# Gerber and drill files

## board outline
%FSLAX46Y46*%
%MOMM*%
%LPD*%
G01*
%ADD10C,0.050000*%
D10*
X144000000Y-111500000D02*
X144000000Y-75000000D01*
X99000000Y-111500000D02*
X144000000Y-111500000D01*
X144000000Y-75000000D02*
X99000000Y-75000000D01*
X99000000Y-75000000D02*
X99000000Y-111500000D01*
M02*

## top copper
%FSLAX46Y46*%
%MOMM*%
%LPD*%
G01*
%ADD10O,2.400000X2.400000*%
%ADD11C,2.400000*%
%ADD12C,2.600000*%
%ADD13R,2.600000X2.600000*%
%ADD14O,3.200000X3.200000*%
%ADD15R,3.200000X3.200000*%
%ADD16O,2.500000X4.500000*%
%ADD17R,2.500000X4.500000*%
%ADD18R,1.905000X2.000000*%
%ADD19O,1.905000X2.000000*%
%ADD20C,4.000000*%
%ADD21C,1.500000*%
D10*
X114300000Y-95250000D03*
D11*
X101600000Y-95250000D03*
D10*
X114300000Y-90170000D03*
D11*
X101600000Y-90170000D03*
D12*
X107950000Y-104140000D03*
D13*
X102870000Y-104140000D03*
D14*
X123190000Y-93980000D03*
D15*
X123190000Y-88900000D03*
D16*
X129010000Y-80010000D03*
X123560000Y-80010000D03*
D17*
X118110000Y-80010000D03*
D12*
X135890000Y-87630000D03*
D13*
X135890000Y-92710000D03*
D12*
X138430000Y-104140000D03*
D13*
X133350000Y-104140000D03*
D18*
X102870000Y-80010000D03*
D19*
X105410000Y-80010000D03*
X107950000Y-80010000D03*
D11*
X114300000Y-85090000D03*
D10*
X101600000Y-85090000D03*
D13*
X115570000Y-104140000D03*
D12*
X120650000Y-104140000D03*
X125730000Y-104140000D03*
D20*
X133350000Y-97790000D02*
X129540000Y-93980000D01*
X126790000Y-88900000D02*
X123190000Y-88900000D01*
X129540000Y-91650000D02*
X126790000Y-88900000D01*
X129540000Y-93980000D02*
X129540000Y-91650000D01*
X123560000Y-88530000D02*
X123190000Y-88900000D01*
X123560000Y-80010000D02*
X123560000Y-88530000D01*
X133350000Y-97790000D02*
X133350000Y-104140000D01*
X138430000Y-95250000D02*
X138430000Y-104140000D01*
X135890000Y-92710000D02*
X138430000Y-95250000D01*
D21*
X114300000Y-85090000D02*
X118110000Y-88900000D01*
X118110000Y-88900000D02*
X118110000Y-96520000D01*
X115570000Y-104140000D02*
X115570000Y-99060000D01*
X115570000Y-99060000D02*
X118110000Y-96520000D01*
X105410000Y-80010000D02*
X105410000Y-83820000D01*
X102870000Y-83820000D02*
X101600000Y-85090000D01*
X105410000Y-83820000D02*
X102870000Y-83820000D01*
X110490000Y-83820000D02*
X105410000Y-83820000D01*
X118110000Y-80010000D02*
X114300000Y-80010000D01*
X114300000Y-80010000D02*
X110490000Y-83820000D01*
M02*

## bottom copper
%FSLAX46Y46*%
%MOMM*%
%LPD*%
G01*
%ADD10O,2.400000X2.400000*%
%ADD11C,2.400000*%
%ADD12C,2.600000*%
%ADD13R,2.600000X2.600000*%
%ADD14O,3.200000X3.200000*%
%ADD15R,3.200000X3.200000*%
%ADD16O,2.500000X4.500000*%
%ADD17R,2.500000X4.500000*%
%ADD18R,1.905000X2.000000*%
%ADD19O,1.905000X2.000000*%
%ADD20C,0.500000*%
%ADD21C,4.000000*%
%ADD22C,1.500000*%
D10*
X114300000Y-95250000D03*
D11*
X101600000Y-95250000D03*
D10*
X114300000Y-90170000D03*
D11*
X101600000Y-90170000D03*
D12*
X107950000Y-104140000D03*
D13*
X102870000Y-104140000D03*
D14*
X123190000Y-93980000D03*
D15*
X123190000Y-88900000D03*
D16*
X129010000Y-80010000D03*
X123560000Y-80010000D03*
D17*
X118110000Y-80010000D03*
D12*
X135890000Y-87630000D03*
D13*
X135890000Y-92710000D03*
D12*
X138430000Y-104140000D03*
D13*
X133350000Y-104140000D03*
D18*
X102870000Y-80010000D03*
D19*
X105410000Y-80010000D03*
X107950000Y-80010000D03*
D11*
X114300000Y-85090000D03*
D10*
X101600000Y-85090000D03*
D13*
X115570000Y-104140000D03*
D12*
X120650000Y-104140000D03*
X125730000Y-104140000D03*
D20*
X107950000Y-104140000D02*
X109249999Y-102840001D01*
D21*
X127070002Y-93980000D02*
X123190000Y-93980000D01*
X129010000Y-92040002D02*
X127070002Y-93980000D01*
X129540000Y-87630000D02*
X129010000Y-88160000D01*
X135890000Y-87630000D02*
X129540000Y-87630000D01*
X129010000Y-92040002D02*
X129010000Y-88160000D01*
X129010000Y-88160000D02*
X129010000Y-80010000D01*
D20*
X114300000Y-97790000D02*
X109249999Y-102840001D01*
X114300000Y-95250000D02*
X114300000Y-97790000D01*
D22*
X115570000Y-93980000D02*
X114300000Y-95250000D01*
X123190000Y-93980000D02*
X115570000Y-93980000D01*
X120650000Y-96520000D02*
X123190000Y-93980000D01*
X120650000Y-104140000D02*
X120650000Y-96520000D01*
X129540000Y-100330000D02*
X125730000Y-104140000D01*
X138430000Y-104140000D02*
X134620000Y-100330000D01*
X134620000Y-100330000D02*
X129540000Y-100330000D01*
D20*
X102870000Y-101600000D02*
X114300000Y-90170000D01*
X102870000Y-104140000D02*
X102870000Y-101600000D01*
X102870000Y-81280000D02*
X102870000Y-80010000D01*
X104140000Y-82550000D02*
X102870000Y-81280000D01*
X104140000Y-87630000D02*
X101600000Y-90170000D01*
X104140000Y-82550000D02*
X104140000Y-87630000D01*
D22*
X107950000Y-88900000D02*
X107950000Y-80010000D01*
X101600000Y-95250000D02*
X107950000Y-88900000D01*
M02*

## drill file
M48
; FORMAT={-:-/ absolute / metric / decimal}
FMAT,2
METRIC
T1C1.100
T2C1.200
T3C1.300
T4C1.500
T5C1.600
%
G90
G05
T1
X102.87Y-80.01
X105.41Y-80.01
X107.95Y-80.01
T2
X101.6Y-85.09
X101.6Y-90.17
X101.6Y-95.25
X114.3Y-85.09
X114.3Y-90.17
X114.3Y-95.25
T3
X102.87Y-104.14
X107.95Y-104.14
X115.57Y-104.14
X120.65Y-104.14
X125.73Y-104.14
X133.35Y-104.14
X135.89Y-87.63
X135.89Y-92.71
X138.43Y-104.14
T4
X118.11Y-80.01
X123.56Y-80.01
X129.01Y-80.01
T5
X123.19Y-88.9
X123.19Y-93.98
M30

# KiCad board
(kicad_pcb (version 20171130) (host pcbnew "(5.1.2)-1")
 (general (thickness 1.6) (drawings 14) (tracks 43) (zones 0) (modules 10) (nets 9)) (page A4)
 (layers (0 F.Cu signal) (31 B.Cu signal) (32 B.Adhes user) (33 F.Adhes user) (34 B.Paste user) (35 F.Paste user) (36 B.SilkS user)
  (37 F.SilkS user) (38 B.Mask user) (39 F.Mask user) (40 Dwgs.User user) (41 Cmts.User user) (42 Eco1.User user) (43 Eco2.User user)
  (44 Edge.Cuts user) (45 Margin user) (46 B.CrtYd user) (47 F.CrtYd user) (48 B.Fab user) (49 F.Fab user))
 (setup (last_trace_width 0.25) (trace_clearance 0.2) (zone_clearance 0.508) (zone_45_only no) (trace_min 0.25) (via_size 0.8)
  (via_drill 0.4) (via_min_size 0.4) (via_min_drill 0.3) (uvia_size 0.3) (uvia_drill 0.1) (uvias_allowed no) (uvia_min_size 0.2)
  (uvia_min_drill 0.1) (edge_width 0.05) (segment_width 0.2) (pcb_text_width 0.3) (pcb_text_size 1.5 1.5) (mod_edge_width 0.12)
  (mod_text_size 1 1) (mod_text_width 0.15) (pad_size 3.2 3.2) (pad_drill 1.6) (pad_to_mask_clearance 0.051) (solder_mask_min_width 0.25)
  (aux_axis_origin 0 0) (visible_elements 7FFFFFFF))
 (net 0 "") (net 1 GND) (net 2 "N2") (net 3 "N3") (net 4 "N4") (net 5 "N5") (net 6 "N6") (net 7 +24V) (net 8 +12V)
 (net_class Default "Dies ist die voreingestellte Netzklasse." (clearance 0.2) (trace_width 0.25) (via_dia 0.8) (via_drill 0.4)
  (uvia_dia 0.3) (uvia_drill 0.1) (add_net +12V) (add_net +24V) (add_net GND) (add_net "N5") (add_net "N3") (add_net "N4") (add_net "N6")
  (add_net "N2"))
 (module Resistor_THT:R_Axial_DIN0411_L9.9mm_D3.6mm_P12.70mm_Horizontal (layer F.Cu) (at 101.6 95.25)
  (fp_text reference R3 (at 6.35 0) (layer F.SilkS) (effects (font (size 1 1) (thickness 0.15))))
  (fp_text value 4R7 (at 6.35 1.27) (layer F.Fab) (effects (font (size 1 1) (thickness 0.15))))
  (pad 2 thru_hole oval (at 12.7 0) (size 2.4 2.4) (drill 1.2) (layers *.Cu *.Mask) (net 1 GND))
  (pad 1 thru_hole circle (at 0 0) (size 2.4 2.4) (drill 1.2) (layers *.Cu *.Mask) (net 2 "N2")))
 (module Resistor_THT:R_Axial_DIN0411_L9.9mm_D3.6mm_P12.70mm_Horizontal (layer F.Cu) (at 101.6 90.17)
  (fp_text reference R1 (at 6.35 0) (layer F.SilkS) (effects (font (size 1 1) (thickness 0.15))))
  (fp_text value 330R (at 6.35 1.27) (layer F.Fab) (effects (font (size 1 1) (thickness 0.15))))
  (pad 2 thru_hole oval (at 12.7 0) (size 2.4 2.4) (drill 1.2) (layers *.Cu *.Mask) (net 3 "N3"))
  (pad 1 thru_hole circle (at 0 0) (size 2.4 2.4) (drill 1.2) (layers *.Cu *.Mask) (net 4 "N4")))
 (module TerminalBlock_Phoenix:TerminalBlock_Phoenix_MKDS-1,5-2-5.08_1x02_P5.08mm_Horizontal (layer F.Cu) (at 102.87 104.14)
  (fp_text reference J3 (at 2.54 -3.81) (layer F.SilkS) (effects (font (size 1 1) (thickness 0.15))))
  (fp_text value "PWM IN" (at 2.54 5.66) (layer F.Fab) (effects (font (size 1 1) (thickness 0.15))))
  (pad 2 thru_hole circle (at 5.08 0) (size 2.6 2.6) (drill 1.3) (layers *.Cu *.Mask) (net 1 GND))
  (pad 1 thru_hole rect (at 0 0) (size 2.6 2.6) (drill 1.3) (layers *.Cu *.Mask) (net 3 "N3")))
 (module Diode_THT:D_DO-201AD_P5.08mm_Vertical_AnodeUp (layer F.Cu) (at 123.19 88.9 270)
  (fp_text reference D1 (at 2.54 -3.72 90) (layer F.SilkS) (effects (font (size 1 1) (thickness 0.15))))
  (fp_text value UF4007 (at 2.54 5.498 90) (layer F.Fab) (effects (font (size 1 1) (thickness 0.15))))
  (pad 2 thru_hole oval (at 5.08 0 270) (size 3.2 3.2) (drill 1.6) (layers *.Cu *.Mask) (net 1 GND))
  (pad 1 thru_hole rect (at 0 0 270) (size 3.2 3.2) (drill 1.6) (layers *.Cu *.Mask) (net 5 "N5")))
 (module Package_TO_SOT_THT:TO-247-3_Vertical (layer F.Cu) (at 118.11 80.01)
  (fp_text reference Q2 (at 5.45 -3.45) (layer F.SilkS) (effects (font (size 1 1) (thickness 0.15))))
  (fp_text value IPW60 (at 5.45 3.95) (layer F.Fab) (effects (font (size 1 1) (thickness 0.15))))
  (pad 3 thru_hole oval (at 10.9 0) (size 2.5 4.5) (drill 1.5) (layers *.Cu *.Mask) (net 1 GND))
  (pad 2 thru_hole oval (at 5.45 0) (size 2.5 4.5) (drill 1.5) (layers *.Cu *.Mask) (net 5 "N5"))
  (pad 1 thru_hole rect (at 0 0) (size 2.5 4.5) (drill 1.5) (layers *.Cu *.Mask) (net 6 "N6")))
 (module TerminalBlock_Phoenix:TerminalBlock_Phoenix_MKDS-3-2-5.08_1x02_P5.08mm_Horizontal (layer F.Cu) (at 135.89 92.71 90)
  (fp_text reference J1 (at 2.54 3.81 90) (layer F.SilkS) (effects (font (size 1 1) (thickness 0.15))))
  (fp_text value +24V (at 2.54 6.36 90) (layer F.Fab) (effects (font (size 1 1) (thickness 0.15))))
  (pad 2 thru_hole circle (at 5.08 0 90) (size 2.6 2.6) (drill 1.3) (layers *.Cu *.Mask) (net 1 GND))
  (pad 1 thru_hole rect (at 0 0 90) (size 2.6 2.6) (drill 1.3) (layers *.Cu *.Mask) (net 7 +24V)))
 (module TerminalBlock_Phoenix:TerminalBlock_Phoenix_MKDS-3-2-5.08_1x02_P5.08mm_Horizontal (layer F.Cu) (at 133.35 104.14)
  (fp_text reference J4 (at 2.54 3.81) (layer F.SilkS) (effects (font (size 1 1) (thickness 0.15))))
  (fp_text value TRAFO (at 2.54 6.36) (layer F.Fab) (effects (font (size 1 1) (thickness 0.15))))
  (pad 2 thru_hole circle (at 5.08 0) (size 2.6 2.6) (drill 1.3) (layers *.Cu *.Mask) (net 7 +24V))
  (pad 1 thru_hole rect (at 0 0) (size 2.6 2.6) (drill 1.3) (layers *.Cu *.Mask) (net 5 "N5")))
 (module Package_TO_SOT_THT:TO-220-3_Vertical (layer F.Cu) (at 102.87 80.01)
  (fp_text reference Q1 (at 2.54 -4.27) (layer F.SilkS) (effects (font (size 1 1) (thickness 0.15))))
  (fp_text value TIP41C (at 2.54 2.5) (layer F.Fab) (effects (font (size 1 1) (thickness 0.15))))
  (pad 1 thru_hole rect (at 0 0) (size 1.905 2) (drill 1.1) (layers *.Cu *.Mask) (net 4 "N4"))
  (pad 2 thru_hole oval (at 2.54 0) (size 1.905 2) (drill 1.1) (layers *.Cu *.Mask) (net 6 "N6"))
  (pad 3 thru_hole oval (at 5.08 0) (size 1.905 2) (drill 1.1) (layers *.Cu *.Mask) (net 2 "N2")))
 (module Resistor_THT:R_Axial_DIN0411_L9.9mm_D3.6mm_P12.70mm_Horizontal (layer F.Cu) (at 114.3 85.09 180)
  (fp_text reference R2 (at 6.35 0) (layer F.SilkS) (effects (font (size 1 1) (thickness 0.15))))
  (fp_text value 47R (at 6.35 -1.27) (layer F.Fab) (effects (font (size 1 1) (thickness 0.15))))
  (pad 1 thru_hole circle (at 0 0 180) (size 2.4 2.4) (drill 1.2) (layers *.Cu *.Mask) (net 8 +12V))
  (pad 2 thru_hole oval (at 12.7 0 180) (size 2.4 2.4) (drill 1.2) (layers *.Cu *.Mask) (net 6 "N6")))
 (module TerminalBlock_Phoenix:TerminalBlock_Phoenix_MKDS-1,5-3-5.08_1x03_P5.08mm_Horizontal (layer F.Cu) (at 115.57 104.14)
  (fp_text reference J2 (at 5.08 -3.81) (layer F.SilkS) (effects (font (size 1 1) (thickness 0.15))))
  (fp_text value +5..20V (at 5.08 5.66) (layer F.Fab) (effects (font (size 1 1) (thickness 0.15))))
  (pad 1 thru_hole rect (at 0 0) (size 2.6 2.6) (drill 1.3) (layers *.Cu *.Mask) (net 8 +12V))
  (pad 2 thru_hole circle (at 5.08 0) (size 2.6 2.6) (drill 1.3) (layers *.Cu *.Mask) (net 1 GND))
  (pad 3 thru_hole circle (at 10.16 0) (size 2.6 2.6) (drill 1.3) (layers *.Cu *.Mask) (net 7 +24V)))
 (gr_line (start 144 111.5) (end 144 75) (layer Edge.Cuts) (width 0.05))
 (gr_line (start 99 111.5) (end 144 111.5) (layer Edge.Cuts) (width 0.05))
 (gr_line (start 144 75) (end 99 75) (layer Edge.Cuts) (width 0.05))
 (gr_line (start 99 75) (end 99 111.5) (layer Edge.Cuts) (width 0.05))
 (segment (start 133.35 97.79) (end 129.54 93.98) (width 4) (layer F.Cu) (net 5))
 (segment (start 126.79 88.9) (end 123.19 88.9) (width 4) (layer F.Cu) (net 5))
 (segment (start 129.54 91.65) (end 126.79 88.9) (width 4) (layer F.Cu) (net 5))
 (segment (start 129.54 93.98) (end 129.54 91.65) (width 4) (layer F.Cu) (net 5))
 (segment (start 123.56 88.53) (end 123.19 88.9) (width 4) (layer F.Cu) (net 5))
 (segment (start 123.56 80.01) (end 123.56 88.53) (width 4) (layer F.Cu) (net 5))
 (segment (start 133.35 97.79) (end 133.35 104.14) (width 4) (layer F.Cu) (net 5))
 (segment (start 107.95 104.14) (end 109.249999 102.840001) (width 0.5) (layer B.Cu) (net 1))
 (segment (start 127.070002 93.98) (end 123.19 93.98) (width 4) (layer B.Cu) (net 1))
 (segment (start 129.01 92.040002) (end 127.070002 93.98) (width 4) (layer B.Cu) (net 1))
 (segment (start 129.54 87.63) (end 129.01 88.16) (width 4) (layer B.Cu) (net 1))
 (segment (start 135.89 87.63) (end 129.54 87.63) (width 4) (layer B.Cu) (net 1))
 (segment (start 129.01 92.040002) (end 129.01 88.16) (width 4) (layer B.Cu) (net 1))
 (segment (start 129.01 88.16) (end 129.01 80.01) (width 4) (layer B.Cu) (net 1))
 (segment (start 114.3 97.79) (end 109.249999 102.840001) (width 0.5) (layer B.Cu) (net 1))
 (segment (start 114.3 95.25) (end 114.3 97.79) (width 0.5) (layer B.Cu) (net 1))
 (segment (start 115.57 93.98) (end 114.3 95.25) (width 1.5) (layer B.Cu) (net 1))
 (segment (start 123.19 93.98) (end 115.57 93.98) (width 1.5) (layer B.Cu) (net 1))
 (segment (start 120.65 96.52) (end 123.19 93.98) (width 1.5) (layer B.Cu) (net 1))
 (segment (start 120.65 104.14) (end 120.65 96.52) (width 1.5) (layer B.Cu) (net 1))
 (segment (start 138.43 95.25) (end 138.43 104.14) (width 4) (layer F.Cu) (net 7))
 (segment (start 135.89 92.71) (end 138.43 95.25) (width 4) (layer F.Cu) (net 7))
 (segment (start 129.54 100.33) (end 125.73 104.14) (width 1.5) (layer B.Cu) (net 7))
 (segment (start 138.43 104.14) (end 134.62 100.33) (width 1.5) (layer B.Cu) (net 7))
 (segment (start 134.62 100.33) (end 129.54 100.33) (width 1.5) (layer B.Cu) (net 7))
 (segment (start 114.3 85.09) (end 118.11 88.9) (width 1.5) (layer F.Cu) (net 8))
 (segment (start 118.11 88.9) (end 118.11 96.52) (width 1.5) (layer F.Cu) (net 8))
 (segment (start 115.57 104.14) (end 115.57 99.06) (width 1.5) (layer F.Cu) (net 8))
 (segment (start 115.57 99.06) (end 118.11 96.52) (width 1.5) (layer F.Cu) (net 8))
 (segment (start 102.87 101.6) (end 114.3 90.17) (width 0.5) (layer B.Cu) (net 3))
 (segment (start 102.87 104.14) (end 102.87 101.6) (width 0.5) (layer B.Cu) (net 3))
 (segment (start 102.87 81.28) (end 102.87 80.01) (width 0.5) (layer B.Cu) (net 4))
 (segment (start 104.14 82.55) (end 102.87 81.28) (width 0.5) (layer B.Cu) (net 4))
 (segment (start 104.14 87.63) (end 101.6 90.17) (width 0.5) (layer B.Cu) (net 4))
 (segment (start 104.14 82.55) (end 104.14 87.63) (width 0.5) (layer B.Cu) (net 4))
 (segment (start 105.41 80.01) (end 105.41 83.82) (width 1.5) (layer F.Cu) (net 6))
 (segment (start 102.87 83.82) (end 101.6 85.09) (width 1.5) (layer F.Cu) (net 6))
 (segment (start 105.41 83.82) (end 102.87 83.82) (width 1.5) (layer F.Cu) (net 6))
 (segment (start 110.49 83.82) (end 105.41 83.82) (width 1.5) (layer F.Cu) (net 6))
 (segment (start 118.11 80.01) (end 114.3 80.01) (width 1.5) (layer F.Cu) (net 6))
 (segment (start 114.3 80.01) (end 110.49 83.82) (width 1.5) (layer F.Cu) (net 6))
 (segment (start 107.95 88.9) (end 107.95 80.01) (width 1.5) (layer B.Cu) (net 2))
 (segment (start 101.6 95.25) (end 107.95 88.9) (width 1.5) (layer B.Cu) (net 2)))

